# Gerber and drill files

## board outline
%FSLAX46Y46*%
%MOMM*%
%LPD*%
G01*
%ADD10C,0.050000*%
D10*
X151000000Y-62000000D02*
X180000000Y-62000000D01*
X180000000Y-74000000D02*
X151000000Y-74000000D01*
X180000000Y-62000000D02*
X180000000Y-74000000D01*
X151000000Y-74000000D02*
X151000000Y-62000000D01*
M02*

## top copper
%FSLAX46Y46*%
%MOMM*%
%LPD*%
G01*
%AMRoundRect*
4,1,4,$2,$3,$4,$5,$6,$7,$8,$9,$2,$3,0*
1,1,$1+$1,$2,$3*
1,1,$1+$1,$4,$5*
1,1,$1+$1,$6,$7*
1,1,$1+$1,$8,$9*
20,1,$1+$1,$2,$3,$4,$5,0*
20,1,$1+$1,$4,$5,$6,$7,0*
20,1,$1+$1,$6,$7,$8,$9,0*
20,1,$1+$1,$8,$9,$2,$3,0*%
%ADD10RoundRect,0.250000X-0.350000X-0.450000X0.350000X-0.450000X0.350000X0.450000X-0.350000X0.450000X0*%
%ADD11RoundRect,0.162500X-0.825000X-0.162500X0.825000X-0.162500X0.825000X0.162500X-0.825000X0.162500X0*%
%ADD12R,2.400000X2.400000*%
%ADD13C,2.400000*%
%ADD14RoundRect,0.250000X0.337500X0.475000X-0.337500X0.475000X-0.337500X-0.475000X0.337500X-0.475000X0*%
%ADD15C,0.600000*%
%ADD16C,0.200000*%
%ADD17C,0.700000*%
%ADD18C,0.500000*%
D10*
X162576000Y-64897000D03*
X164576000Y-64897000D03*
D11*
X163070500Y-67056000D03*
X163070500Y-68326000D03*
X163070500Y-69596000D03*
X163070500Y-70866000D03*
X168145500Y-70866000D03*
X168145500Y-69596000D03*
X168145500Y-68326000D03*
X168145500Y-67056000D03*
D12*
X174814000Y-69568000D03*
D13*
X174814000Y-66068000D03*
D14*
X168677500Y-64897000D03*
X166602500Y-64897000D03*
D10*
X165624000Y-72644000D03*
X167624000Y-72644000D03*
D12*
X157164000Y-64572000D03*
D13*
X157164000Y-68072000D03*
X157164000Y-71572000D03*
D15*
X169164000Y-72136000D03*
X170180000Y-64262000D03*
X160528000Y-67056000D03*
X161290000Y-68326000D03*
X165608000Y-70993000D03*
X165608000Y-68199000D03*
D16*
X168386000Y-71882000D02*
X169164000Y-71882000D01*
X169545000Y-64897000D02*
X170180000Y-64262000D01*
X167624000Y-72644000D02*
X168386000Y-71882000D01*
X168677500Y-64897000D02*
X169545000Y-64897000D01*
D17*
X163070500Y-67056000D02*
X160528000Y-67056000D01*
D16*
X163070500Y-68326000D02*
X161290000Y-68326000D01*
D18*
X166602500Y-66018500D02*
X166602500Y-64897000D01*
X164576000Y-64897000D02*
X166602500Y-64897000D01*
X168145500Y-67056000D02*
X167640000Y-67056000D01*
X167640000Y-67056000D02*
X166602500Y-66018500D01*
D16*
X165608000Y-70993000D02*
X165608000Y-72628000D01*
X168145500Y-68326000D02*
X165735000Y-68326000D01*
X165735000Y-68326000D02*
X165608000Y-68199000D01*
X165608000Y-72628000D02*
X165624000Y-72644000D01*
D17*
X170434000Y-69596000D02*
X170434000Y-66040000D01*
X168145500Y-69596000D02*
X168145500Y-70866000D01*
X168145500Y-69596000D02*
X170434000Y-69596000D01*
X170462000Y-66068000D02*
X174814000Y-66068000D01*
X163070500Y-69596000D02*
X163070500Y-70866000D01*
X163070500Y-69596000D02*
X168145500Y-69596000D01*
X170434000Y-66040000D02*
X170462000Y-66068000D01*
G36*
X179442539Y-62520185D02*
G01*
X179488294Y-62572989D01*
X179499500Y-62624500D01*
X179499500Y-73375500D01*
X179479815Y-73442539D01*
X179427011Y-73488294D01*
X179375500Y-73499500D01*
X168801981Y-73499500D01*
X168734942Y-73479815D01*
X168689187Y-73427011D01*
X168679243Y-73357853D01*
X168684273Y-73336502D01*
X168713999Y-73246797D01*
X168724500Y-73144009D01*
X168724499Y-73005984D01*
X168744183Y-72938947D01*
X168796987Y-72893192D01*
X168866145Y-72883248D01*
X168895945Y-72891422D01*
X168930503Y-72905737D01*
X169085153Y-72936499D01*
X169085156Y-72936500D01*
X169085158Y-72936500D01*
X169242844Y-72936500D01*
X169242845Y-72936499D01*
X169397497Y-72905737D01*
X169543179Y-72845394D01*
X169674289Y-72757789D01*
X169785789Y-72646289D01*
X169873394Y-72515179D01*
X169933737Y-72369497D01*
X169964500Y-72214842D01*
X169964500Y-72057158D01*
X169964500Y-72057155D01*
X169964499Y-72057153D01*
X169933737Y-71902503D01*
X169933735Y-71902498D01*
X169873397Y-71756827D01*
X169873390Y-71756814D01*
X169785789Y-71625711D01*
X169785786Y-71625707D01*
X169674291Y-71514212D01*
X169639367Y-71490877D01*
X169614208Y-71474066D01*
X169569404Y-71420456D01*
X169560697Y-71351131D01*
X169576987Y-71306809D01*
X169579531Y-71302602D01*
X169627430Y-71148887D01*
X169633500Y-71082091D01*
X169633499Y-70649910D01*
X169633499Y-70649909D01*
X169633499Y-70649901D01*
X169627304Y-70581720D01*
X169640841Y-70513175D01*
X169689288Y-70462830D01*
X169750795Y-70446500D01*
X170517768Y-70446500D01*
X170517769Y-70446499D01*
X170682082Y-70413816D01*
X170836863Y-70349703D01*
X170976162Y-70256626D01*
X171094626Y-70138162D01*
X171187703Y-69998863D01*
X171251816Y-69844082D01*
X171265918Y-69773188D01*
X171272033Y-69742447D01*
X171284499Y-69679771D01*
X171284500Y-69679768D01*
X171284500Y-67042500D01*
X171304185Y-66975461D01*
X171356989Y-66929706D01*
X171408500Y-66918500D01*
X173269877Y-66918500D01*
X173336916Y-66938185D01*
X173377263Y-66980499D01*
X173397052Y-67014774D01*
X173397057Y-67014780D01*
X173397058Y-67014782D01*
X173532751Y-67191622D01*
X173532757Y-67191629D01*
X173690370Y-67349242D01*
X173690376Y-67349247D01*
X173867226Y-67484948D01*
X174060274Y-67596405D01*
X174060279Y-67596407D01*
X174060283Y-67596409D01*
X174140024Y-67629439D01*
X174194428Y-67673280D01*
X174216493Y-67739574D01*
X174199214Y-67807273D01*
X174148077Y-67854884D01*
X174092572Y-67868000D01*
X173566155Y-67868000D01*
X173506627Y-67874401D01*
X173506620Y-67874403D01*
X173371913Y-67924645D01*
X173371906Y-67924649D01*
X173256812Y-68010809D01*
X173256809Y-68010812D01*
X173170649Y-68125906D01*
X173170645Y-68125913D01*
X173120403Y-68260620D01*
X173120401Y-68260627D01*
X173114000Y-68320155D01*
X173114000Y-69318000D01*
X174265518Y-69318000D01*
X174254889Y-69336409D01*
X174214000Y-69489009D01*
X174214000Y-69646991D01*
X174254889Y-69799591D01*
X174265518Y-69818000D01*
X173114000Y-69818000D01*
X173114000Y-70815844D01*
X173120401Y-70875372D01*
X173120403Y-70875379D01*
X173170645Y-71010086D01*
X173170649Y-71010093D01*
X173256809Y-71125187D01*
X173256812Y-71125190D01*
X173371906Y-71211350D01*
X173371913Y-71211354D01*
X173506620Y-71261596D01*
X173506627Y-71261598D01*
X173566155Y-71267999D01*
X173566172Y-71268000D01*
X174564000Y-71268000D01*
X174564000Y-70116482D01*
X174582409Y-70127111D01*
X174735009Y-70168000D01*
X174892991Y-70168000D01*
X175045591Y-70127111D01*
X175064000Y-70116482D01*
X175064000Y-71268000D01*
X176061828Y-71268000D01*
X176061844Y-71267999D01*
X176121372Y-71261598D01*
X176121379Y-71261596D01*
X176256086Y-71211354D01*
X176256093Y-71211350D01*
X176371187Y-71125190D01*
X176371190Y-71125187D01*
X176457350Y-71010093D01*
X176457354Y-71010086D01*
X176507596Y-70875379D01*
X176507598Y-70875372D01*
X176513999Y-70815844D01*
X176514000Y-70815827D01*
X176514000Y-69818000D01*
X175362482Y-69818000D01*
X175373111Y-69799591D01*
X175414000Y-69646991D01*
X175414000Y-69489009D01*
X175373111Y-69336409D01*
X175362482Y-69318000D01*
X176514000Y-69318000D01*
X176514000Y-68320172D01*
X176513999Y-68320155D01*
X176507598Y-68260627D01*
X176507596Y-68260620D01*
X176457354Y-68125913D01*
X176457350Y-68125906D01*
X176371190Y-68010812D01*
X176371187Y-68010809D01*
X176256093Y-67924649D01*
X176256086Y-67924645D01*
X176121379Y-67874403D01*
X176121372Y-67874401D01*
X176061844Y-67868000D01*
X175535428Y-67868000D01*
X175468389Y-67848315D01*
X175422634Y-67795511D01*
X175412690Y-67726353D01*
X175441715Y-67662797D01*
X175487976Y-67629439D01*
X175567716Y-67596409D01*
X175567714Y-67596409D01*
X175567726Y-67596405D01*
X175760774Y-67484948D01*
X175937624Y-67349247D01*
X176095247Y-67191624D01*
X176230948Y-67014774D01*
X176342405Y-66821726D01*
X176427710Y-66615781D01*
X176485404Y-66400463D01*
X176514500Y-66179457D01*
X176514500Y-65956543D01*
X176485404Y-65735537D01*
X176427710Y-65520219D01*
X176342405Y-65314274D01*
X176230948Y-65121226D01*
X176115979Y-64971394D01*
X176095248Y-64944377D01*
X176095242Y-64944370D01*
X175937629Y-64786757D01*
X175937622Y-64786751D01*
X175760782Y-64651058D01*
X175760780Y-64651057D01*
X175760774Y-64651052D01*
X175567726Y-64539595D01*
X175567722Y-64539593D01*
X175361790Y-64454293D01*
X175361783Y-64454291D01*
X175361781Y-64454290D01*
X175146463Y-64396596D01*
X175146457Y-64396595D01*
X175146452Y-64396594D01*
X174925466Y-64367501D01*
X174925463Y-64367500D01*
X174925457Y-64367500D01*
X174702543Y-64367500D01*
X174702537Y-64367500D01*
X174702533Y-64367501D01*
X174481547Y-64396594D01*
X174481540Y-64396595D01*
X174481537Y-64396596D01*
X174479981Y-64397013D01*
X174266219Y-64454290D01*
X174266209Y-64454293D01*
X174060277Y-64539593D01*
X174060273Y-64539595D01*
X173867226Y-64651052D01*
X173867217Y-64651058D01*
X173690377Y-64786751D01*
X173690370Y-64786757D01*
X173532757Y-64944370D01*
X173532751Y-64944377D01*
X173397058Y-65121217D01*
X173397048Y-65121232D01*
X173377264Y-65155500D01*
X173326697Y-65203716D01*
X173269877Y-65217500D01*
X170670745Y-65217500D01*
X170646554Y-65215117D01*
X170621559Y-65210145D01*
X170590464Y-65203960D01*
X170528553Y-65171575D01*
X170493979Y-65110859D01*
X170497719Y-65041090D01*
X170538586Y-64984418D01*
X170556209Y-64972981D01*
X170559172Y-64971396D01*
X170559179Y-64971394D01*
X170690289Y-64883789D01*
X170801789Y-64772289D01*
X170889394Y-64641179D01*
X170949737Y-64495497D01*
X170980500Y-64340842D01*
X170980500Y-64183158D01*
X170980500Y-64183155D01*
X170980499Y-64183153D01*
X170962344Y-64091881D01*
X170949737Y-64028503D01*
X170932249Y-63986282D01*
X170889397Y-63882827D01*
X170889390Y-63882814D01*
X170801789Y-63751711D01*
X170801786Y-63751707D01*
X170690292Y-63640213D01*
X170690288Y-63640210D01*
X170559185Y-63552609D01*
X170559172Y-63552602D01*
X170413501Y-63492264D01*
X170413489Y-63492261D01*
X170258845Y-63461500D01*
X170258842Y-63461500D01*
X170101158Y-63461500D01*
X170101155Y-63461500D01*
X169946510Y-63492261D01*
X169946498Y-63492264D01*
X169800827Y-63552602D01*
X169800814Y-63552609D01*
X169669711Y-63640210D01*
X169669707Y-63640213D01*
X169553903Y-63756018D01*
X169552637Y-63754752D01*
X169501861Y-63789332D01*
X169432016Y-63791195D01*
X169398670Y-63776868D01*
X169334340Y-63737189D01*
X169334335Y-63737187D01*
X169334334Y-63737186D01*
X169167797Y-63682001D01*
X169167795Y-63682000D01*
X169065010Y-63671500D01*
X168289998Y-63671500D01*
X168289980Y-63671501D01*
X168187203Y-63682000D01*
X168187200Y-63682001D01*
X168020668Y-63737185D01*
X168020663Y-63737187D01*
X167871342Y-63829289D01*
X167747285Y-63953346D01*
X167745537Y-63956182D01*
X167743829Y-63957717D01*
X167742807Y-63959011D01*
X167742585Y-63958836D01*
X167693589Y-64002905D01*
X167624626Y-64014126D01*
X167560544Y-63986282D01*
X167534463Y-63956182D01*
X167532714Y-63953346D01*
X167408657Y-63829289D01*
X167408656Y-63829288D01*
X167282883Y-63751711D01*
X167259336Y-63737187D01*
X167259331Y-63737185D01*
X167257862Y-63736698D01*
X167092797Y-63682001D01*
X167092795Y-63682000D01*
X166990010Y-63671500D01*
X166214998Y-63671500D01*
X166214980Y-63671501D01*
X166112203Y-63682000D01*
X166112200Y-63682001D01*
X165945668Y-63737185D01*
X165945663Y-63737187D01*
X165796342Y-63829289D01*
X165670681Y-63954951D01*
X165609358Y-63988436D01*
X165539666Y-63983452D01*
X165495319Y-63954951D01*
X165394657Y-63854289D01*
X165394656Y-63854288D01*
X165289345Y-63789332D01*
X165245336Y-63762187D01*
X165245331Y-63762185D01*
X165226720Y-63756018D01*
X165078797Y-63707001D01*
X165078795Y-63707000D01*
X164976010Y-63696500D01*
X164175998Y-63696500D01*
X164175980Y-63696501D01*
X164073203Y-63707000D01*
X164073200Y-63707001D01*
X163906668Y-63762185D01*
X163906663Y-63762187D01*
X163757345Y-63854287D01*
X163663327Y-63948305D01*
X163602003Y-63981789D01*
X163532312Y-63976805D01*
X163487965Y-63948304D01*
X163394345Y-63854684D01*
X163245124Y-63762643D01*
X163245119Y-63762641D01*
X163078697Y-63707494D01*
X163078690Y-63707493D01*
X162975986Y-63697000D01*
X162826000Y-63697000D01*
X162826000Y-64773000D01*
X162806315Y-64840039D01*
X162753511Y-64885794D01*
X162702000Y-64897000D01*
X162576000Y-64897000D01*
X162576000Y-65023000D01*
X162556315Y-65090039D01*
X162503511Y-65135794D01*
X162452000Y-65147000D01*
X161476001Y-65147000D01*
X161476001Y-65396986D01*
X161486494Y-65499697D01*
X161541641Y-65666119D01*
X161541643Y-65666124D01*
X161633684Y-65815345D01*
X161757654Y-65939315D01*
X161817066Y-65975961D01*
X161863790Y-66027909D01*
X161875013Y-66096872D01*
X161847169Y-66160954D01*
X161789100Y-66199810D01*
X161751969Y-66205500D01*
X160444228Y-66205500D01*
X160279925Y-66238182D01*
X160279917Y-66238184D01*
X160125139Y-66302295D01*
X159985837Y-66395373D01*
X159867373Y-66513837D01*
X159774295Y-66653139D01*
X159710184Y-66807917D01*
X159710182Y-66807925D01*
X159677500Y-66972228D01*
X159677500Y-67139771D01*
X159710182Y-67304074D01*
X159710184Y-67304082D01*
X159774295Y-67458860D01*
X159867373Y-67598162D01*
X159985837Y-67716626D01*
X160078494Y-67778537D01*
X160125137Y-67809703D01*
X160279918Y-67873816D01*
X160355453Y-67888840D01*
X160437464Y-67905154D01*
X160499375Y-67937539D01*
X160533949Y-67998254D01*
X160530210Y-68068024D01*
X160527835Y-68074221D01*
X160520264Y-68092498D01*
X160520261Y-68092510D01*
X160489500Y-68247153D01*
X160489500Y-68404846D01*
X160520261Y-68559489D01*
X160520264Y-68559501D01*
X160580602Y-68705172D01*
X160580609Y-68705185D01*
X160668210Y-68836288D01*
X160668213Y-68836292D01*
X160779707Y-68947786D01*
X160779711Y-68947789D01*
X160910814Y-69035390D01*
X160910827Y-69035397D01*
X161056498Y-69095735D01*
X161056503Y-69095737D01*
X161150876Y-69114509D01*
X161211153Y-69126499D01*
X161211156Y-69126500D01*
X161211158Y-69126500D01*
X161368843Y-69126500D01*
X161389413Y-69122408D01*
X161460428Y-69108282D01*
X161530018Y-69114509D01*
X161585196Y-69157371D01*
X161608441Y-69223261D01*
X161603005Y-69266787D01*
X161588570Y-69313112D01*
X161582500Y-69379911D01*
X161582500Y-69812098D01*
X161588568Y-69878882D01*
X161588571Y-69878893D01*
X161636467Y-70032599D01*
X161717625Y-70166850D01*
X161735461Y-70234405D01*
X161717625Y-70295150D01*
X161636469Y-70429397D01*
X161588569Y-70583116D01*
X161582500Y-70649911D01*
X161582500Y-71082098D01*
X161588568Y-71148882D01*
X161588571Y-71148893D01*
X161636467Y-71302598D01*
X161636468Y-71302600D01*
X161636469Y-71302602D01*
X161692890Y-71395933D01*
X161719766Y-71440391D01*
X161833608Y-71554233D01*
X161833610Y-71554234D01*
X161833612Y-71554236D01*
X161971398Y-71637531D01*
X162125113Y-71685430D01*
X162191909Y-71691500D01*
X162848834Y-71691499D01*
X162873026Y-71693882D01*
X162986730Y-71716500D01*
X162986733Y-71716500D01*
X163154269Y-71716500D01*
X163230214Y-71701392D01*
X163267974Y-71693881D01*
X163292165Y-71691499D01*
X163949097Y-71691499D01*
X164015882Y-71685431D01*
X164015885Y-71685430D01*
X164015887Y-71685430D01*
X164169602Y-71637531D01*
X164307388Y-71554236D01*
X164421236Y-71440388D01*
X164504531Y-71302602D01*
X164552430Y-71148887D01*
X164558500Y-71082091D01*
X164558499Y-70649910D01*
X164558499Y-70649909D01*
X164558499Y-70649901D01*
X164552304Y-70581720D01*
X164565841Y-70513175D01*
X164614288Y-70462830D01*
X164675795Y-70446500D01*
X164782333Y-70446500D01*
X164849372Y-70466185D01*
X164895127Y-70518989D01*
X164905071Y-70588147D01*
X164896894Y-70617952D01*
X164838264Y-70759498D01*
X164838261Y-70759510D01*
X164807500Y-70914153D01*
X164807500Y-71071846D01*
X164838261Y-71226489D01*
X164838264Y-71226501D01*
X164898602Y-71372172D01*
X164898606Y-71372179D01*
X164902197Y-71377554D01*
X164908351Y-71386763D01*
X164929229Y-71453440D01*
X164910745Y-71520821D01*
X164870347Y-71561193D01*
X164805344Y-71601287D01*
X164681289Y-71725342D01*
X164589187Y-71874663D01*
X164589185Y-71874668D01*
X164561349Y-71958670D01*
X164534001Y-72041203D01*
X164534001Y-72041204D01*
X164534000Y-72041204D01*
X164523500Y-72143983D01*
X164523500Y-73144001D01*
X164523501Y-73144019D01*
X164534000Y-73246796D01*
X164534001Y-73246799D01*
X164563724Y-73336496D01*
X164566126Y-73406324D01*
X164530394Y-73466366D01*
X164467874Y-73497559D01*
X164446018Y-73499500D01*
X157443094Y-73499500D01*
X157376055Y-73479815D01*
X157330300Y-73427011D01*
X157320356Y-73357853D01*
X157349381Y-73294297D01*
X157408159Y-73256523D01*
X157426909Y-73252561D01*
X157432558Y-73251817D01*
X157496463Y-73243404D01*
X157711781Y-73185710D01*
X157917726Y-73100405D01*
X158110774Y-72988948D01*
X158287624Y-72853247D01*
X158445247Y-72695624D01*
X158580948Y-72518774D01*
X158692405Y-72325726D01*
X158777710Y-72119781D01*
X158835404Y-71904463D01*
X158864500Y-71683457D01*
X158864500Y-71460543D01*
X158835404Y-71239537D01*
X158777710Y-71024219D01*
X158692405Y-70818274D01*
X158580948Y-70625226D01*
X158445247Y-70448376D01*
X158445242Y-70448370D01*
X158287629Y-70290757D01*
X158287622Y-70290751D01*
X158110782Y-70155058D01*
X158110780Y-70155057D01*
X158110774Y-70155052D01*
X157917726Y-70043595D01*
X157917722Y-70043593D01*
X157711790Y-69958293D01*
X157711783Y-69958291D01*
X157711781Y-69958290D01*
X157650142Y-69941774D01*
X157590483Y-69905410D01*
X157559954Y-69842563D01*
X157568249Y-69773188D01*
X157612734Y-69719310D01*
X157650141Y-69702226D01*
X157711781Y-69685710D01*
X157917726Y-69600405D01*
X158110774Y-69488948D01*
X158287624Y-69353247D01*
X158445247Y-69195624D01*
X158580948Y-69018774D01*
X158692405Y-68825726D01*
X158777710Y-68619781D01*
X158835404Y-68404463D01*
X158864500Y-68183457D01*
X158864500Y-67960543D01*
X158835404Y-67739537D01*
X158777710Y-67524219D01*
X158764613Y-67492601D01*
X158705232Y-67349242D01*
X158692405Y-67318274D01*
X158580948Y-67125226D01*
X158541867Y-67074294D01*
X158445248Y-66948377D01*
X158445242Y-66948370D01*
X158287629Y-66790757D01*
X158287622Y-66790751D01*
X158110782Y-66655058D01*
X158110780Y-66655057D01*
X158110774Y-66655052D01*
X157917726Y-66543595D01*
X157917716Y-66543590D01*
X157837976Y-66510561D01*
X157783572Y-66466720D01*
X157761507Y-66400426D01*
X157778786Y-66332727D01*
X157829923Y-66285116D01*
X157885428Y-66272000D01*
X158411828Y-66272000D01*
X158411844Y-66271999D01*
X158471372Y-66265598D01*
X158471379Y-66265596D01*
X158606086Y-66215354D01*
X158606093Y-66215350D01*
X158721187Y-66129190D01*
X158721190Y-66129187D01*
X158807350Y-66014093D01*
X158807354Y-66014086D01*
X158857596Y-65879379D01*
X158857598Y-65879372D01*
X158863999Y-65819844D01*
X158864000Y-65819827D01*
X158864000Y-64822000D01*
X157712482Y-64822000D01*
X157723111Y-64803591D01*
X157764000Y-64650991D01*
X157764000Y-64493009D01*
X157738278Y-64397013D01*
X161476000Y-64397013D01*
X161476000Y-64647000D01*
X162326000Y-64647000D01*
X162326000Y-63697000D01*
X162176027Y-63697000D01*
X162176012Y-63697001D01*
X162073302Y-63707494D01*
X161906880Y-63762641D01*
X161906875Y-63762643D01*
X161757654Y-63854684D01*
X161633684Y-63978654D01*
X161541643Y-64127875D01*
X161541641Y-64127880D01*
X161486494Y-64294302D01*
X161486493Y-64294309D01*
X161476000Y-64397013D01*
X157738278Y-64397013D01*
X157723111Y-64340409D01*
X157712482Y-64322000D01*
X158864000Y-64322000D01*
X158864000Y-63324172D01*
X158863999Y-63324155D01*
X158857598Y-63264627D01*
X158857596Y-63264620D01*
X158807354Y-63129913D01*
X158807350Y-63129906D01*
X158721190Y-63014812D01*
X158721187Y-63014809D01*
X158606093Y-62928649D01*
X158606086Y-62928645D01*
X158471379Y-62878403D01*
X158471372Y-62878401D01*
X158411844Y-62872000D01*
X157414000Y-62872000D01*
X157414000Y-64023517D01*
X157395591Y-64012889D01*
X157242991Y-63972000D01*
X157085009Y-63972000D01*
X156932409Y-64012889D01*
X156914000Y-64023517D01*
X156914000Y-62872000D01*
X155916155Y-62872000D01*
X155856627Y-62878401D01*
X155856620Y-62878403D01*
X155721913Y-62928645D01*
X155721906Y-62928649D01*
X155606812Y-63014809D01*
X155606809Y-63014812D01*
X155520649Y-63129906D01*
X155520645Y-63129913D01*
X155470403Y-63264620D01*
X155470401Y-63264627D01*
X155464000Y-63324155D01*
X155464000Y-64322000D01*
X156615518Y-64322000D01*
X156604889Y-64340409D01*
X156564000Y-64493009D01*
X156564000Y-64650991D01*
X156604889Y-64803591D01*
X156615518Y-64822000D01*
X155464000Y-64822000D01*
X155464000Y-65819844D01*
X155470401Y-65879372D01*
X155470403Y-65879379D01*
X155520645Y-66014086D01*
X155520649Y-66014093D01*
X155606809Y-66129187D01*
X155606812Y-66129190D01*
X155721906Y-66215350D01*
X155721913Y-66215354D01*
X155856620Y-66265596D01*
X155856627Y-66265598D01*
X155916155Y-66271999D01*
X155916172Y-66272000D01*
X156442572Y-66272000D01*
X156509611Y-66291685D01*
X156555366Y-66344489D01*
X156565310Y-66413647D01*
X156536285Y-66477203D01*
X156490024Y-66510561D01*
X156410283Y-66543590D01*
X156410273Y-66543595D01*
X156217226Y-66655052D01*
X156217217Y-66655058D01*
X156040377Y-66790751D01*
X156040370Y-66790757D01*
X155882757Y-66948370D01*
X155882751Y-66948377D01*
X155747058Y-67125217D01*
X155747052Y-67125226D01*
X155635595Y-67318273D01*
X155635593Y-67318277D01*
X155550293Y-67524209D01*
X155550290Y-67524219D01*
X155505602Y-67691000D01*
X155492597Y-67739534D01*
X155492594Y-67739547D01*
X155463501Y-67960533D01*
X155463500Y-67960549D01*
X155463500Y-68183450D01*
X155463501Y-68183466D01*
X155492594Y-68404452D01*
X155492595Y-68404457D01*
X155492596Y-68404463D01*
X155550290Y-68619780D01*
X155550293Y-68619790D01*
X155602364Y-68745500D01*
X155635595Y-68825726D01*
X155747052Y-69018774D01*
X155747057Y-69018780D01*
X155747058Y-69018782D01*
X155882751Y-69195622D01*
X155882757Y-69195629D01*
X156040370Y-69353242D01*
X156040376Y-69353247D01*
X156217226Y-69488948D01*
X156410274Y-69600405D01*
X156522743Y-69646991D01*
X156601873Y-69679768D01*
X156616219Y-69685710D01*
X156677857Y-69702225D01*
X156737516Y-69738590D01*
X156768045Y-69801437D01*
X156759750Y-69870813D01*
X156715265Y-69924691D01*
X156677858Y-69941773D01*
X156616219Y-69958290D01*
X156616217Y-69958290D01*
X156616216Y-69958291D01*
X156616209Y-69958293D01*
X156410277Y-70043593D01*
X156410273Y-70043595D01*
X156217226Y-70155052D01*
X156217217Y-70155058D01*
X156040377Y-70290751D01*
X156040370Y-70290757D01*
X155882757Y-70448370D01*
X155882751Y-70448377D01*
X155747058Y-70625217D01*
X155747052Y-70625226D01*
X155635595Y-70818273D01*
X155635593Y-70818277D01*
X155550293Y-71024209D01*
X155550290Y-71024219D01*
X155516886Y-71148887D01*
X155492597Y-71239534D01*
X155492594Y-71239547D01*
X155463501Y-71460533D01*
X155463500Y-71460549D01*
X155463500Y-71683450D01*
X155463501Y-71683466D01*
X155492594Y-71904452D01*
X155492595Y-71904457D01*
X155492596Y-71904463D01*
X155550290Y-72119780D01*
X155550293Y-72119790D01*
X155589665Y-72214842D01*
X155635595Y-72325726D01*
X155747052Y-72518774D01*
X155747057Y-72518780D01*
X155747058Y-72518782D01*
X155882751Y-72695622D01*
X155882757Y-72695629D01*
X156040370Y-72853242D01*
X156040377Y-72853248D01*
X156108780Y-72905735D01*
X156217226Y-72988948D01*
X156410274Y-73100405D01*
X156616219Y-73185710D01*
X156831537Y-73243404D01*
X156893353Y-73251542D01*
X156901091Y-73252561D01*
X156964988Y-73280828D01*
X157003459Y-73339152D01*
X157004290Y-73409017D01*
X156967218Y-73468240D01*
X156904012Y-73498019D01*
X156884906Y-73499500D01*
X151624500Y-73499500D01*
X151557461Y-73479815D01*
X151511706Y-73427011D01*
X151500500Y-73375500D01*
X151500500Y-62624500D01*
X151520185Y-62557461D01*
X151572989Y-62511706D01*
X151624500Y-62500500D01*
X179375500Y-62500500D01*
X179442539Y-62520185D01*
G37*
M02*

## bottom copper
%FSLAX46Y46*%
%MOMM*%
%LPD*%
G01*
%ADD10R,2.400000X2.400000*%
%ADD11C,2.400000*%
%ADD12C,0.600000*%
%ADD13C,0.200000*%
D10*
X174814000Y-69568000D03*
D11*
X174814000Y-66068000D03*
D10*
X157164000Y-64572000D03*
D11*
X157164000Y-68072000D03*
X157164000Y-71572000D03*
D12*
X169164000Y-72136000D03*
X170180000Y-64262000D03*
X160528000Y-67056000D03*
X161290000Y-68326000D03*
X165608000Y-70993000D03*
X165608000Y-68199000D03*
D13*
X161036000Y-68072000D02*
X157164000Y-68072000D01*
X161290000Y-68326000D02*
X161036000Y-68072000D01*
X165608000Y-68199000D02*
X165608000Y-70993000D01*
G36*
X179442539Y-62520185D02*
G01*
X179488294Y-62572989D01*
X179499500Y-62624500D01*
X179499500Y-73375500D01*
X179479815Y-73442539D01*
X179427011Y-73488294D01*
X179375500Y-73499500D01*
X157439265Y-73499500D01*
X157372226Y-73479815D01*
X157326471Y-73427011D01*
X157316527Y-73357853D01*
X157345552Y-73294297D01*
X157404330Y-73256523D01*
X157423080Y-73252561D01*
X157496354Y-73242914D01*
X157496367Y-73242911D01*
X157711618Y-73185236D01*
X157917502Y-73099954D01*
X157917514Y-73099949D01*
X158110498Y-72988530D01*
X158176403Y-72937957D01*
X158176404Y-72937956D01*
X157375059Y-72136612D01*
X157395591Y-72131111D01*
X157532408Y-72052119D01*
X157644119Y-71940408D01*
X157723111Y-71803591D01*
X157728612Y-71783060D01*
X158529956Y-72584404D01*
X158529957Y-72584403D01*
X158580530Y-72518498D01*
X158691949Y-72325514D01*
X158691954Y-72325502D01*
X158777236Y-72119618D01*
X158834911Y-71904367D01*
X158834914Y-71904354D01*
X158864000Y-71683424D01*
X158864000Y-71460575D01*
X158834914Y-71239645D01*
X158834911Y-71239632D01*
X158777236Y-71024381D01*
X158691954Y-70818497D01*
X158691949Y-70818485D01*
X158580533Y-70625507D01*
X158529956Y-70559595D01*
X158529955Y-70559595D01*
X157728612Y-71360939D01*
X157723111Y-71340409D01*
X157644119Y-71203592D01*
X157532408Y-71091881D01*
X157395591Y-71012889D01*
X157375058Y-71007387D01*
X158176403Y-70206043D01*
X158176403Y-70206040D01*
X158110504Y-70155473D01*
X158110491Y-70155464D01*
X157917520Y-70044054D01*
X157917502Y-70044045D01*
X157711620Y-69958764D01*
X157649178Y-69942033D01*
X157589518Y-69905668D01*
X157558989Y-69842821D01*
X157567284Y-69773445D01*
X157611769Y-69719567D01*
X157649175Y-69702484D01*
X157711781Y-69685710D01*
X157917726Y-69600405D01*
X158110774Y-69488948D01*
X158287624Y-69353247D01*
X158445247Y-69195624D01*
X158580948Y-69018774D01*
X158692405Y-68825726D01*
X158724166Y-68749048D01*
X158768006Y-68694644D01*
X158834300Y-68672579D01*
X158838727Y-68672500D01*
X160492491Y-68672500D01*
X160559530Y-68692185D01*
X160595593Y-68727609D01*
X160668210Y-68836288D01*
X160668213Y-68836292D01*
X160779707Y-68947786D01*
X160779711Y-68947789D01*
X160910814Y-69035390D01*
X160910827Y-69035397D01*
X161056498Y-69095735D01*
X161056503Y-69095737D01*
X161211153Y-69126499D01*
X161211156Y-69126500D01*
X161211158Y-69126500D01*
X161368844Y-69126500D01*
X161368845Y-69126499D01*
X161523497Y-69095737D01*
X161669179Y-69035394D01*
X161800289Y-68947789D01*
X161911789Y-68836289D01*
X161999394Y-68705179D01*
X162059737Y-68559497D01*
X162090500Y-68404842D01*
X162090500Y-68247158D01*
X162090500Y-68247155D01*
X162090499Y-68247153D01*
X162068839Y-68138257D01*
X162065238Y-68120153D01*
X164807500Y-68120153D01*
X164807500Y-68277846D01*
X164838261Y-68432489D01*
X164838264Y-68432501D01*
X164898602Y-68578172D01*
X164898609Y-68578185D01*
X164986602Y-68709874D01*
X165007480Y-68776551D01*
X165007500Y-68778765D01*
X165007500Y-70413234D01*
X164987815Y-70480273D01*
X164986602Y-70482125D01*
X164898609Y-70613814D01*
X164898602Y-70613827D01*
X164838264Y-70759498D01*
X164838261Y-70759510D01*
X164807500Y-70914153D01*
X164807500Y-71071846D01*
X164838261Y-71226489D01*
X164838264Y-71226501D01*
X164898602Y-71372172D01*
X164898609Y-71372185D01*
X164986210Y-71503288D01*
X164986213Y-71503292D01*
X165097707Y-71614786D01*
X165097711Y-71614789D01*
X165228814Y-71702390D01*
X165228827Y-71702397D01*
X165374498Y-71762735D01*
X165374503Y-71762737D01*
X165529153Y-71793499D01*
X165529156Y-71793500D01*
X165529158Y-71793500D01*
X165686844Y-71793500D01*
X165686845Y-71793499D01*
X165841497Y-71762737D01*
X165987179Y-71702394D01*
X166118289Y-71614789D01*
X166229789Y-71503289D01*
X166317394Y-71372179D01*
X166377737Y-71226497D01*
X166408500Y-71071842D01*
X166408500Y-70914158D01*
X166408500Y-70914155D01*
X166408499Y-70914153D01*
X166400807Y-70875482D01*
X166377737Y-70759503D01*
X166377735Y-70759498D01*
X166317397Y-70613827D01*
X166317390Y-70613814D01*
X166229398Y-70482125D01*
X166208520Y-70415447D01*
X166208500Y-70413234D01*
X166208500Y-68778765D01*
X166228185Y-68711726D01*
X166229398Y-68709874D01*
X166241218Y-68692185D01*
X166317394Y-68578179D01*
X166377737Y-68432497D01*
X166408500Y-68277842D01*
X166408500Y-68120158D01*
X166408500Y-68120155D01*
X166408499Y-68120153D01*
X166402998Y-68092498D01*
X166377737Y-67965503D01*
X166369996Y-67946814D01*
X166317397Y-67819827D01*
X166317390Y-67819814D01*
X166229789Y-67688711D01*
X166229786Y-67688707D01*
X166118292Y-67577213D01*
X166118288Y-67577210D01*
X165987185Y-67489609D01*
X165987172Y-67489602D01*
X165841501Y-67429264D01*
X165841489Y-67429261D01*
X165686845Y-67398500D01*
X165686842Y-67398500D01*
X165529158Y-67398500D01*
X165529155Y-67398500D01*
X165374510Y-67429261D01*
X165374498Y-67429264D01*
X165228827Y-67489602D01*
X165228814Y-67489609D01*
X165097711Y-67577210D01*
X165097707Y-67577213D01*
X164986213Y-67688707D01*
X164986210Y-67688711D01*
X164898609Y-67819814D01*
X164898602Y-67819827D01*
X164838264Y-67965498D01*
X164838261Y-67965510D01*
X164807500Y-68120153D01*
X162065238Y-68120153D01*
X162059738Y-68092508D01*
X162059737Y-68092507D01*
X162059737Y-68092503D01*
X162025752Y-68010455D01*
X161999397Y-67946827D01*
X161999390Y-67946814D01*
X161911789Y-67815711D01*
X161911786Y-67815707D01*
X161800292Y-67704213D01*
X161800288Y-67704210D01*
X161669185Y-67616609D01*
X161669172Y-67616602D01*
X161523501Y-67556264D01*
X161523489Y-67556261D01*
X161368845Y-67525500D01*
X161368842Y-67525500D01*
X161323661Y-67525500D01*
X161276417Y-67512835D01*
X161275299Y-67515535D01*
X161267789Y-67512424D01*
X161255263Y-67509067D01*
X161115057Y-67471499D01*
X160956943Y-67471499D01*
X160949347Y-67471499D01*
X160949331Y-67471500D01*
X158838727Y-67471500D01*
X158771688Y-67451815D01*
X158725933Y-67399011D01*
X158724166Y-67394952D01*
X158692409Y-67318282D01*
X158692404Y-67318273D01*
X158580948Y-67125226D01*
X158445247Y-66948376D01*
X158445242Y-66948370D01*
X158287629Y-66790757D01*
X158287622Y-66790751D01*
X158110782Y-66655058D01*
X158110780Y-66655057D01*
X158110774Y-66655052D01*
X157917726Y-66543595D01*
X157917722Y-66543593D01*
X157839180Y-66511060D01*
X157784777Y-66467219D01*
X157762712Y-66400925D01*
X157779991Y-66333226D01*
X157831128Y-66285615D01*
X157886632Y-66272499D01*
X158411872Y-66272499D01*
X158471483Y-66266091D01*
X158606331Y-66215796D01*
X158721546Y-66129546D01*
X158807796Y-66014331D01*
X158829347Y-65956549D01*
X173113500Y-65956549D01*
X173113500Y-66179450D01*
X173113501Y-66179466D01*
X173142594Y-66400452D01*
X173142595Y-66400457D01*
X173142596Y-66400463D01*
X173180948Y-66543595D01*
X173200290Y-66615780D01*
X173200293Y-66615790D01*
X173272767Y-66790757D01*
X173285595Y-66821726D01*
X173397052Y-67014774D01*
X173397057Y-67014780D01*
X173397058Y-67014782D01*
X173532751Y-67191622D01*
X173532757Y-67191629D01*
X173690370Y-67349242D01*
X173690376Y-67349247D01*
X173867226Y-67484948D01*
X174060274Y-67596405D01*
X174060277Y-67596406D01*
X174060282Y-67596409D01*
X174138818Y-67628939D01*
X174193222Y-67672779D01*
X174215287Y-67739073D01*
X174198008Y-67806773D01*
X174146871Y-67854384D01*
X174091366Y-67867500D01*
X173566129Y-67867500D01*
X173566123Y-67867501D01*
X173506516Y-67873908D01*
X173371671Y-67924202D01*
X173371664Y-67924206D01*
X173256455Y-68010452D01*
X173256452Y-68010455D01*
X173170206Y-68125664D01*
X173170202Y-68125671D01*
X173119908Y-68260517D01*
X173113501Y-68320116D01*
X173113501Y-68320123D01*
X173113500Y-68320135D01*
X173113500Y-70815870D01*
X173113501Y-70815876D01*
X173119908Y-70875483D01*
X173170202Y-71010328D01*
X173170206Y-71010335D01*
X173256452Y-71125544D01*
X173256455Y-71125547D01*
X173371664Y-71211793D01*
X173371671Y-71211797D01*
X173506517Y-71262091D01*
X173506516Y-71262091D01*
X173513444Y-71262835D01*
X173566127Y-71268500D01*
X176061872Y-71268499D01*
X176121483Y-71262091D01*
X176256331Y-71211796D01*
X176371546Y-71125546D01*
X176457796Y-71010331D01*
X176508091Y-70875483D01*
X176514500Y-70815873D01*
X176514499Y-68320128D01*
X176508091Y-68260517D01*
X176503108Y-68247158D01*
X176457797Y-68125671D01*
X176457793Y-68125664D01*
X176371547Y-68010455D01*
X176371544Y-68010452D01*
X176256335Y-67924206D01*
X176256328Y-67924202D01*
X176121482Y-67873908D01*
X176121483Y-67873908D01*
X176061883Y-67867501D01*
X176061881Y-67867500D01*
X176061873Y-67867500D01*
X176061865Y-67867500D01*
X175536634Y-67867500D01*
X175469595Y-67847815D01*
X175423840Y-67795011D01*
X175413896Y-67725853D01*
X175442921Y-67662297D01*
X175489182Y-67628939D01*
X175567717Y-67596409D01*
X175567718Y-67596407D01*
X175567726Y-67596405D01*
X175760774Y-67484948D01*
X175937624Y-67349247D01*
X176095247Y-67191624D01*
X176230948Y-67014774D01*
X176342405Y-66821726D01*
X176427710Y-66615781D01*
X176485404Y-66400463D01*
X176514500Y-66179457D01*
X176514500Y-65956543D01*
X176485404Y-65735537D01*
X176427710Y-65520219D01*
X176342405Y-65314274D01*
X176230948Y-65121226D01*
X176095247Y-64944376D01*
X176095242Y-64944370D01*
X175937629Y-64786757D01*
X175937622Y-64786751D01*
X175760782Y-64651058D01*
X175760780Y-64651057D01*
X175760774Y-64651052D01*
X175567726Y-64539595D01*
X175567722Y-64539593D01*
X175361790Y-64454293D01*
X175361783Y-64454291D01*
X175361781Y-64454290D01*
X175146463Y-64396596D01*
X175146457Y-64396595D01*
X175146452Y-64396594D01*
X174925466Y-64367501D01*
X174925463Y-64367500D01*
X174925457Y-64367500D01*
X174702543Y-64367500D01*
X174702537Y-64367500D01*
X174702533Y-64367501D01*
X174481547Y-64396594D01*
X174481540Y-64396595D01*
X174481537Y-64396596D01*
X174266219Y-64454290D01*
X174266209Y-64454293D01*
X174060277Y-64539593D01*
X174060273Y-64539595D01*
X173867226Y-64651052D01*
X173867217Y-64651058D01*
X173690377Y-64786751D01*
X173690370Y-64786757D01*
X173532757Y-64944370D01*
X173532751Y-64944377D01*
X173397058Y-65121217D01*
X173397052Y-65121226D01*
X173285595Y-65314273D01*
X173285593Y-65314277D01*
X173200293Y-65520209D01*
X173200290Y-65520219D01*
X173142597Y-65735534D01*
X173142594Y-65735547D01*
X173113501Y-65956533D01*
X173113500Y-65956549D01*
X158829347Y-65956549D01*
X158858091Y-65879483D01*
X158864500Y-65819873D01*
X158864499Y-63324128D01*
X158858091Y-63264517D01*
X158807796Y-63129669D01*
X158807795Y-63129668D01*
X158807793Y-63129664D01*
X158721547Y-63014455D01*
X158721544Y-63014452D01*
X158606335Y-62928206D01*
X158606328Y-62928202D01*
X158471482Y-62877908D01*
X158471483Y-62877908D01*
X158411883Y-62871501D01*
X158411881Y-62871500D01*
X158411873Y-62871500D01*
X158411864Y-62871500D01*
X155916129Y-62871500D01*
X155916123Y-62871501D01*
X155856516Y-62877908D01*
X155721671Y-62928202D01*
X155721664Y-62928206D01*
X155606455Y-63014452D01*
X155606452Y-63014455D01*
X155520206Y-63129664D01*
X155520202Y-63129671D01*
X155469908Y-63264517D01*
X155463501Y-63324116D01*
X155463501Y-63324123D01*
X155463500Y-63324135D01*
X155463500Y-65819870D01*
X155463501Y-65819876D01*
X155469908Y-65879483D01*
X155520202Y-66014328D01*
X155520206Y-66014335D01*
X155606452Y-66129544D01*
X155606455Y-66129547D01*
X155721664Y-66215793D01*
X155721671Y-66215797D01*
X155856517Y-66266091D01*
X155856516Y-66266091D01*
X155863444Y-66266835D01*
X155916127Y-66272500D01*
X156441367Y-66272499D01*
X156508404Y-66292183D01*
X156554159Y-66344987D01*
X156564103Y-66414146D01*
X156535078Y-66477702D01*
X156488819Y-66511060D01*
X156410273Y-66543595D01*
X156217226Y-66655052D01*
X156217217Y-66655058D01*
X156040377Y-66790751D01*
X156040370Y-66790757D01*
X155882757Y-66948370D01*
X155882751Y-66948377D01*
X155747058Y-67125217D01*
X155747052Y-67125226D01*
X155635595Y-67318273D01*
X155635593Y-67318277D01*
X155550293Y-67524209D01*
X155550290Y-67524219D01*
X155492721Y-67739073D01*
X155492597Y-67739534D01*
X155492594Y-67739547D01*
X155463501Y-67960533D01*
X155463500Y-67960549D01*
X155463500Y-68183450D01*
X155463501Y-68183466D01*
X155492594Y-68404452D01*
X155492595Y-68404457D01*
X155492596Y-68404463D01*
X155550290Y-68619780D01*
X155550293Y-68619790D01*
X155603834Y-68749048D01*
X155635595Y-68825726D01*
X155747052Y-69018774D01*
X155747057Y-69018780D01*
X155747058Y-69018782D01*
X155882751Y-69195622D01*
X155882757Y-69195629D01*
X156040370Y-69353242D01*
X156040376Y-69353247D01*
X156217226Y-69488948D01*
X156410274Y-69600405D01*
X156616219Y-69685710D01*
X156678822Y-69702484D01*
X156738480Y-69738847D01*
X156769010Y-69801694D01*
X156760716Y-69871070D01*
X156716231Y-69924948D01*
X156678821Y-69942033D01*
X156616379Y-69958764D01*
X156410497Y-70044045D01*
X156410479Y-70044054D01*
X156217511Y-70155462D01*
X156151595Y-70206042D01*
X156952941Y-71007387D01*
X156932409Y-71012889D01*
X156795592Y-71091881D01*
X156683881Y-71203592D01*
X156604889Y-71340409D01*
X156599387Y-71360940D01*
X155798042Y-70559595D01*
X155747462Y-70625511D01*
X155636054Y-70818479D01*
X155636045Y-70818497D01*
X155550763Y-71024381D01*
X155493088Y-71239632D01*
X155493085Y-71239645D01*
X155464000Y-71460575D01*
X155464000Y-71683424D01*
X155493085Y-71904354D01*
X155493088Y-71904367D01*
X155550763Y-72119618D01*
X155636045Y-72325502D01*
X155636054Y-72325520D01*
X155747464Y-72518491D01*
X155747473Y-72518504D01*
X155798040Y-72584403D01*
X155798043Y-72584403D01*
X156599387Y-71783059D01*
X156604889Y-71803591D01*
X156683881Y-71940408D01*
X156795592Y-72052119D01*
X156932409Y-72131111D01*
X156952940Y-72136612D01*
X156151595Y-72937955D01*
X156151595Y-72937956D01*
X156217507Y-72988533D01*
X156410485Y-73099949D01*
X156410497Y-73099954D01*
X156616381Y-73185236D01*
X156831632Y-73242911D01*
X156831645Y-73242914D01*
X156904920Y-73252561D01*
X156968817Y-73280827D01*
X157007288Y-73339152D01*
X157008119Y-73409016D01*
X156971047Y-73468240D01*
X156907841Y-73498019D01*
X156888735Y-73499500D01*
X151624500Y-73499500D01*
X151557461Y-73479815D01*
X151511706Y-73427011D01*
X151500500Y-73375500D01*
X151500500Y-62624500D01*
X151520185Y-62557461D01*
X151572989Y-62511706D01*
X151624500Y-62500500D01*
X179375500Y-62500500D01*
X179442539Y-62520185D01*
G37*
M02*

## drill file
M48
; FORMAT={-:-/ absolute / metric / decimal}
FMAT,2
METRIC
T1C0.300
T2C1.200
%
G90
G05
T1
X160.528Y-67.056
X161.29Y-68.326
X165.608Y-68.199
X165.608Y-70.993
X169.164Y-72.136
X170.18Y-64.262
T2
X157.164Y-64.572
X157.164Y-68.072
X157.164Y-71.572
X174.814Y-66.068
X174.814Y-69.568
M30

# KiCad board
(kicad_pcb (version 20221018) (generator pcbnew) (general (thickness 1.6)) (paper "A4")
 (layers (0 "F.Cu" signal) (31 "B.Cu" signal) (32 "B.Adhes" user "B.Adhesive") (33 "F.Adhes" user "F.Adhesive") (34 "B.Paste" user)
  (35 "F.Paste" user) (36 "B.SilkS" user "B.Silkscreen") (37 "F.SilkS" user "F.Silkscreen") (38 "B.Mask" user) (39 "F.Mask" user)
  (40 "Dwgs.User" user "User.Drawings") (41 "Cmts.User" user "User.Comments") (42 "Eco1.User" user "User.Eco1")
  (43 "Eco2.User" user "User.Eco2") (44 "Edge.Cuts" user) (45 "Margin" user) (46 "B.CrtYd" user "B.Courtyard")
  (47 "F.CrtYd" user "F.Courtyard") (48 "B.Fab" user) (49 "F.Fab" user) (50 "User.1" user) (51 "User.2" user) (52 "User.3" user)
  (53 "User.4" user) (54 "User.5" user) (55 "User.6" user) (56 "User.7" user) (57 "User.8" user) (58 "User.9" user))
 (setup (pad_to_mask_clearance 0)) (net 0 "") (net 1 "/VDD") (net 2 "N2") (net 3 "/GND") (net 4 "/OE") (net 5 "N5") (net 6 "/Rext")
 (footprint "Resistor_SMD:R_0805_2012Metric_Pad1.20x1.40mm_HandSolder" (layer "F.Cu") (at 163.576 64.897)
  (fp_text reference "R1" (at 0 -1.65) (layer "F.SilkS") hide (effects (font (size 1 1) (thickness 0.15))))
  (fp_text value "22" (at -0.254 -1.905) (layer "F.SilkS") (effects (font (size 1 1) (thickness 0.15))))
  (pad "1" smd roundrect (at -1 0) (size 1.2 1.4) (layers "F.Cu" "F.Paste" "F.Mask") (roundrect_rratio 0.2083333333) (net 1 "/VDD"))
  (pad "2" smd roundrect (at 1 0) (size 1.2 1.4) (layers "F.Cu" "F.Paste" "F.Mask") (roundrect_rratio 0.2083333333) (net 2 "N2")))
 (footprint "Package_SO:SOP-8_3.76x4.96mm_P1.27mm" (layer "F.Cu") (at 165.608 68.961)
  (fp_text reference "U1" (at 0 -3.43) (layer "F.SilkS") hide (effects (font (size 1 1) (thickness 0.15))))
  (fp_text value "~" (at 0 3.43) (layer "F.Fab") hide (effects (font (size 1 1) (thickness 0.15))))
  (pad "1" smd roundrect (at -2.5375 -1.905) (size 1.975 0.65) (layers "F.Cu" "F.Paste" "F.Mask") (roundrect_rratio 0.25) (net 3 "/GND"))
  (pad "2" smd roundrect (at -2.5375 -0.635) (size 1.975 0.65) (layers "F.Cu" "F.Paste" "F.Mask") (roundrect_rratio 0.25) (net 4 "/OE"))
  (pad "3" smd roundrect (at -2.5375 0.635) (size 1.975 0.65) (layers "F.Cu" "F.Paste" "F.Mask") (roundrect_rratio 0.25) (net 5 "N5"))
  (pad "4" smd roundrect (at -2.5375 1.905) (size 1.975 0.65) (layers "F.Cu" "F.Paste" "F.Mask") (roundrect_rratio 0.25) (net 5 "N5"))
  (pad "5" smd roundrect (at 2.5375 1.905) (size 1.975 0.65) (layers "F.Cu" "F.Paste" "F.Mask") (roundrect_rratio 0.25) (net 5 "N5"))
  (pad "6" smd roundrect (at 2.5375 0.635) (size 1.975 0.65) (layers "F.Cu" "F.Paste" "F.Mask") (roundrect_rratio 0.25) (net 5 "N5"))
  (pad "7" smd roundrect (at 2.5375 -0.635) (size 1.975 0.65) (layers "F.Cu" "F.Paste" "F.Mask") (roundrect_rratio 0.25) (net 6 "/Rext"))
  (pad "8" smd roundrect (at 2.5375 -1.905) (size 1.975 0.65) (layers "F.Cu" "F.Paste" "F.Mask") (roundrect_rratio 0.25) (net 2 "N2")))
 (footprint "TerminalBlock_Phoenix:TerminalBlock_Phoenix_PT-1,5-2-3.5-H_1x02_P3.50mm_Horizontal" (layer "F.Cu") (at 174.814 69.568 90)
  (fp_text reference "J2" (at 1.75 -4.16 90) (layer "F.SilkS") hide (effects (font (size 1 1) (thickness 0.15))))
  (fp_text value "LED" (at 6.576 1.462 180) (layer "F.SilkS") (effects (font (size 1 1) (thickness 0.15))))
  (pad "1" thru_hole rect (at 0 0 90) (size 2.4 2.4) (drill 1.2) (layers "*.Cu" "*.Mask") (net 1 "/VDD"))
  (pad "2" thru_hole circle (at 3.5 0 90) (size 2.4 2.4) (drill 1.2) (layers "*.Cu" "*.Mask") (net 5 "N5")))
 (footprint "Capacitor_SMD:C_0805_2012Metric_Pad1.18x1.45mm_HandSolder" (layer "F.Cu") (at 167.64 64.897 180)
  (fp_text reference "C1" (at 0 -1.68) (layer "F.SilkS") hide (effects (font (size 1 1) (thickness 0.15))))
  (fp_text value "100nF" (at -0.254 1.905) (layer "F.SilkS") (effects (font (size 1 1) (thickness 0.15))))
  (pad "1" smd roundrect (at -1.0375 0 180) (size 1.175 1.45) (layers "F.Cu" "F.Paste" "F.Mask") (roundrect_rratio 0.2127659574)
   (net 3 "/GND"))
  (pad "2" smd roundrect (at 1.0375 0 180) (size 1.175 1.45) (layers "F.Cu" "F.Paste" "F.Mask") (roundrect_rratio 0.2127659574) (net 2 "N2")))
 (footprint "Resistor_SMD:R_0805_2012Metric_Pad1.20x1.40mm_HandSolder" (layer "F.Cu") (at 166.624 72.644)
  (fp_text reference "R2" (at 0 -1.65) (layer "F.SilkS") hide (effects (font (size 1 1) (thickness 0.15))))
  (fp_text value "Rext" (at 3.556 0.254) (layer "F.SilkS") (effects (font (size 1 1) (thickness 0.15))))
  (pad "1" smd roundrect (at -1 0) (size 1.2 1.4) (layers "F.Cu" "F.Paste" "F.Mask") (roundrect_rratio 0.2083333333) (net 6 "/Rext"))
  (pad "2" smd roundrect (at 1 0) (size 1.2 1.4) (layers "F.Cu" "F.Paste" "F.Mask") (roundrect_rratio 0.2083333333) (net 3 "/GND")))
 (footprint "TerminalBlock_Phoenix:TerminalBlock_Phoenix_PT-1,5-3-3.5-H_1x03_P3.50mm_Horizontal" (layer "F.Cu") (at 157.164 64.572 -90)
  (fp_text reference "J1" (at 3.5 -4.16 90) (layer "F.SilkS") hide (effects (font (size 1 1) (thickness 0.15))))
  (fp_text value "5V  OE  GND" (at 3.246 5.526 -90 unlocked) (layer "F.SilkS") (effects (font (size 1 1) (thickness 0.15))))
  (pad "1" thru_hole rect (at 0 0 270) (size 2.4 2.4) (drill 1.2) (layers "*.Cu" "*.Mask") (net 1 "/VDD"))
  (pad "2" thru_hole circle (at 3.5 0 270) (size 2.4 2.4) (drill 1.2) (layers "*.Cu" "*.Mask") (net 4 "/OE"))
  (pad "3" thru_hole circle (at 7 0 270) (size 2.4 2.4) (drill 1.2) (layers "*.Cu" "*.Mask") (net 3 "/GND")))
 (gr_line (start 151 62) (end 180 62) (stroke (width 0.05) (type default)) (layer "Edge.Cuts"))
 (gr_line (start 180 74) (end 151 74) (stroke (width 0.05) (type default)) (layer "Edge.Cuts"))
 (gr_line (start 180 62) (end 180 74) (stroke (width 0.05) (type default)) (layer "Edge.Cuts"))
 (gr_line (start 151 74) (end 151 62) (stroke (width 0.05) (type default)) (layer "Edge.Cuts"))
 (segment (start 168.386 71.882) (end 169.164 71.882) (width 0.2) (layer "F.Cu") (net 3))
 (segment (start 169.545 64.897) (end 170.18 64.262) (width 0.2) (layer "F.Cu") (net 3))
 (segment (start 167.624 72.644) (end 168.386 71.882) (width 0.2) (layer "F.Cu") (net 3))
 (segment (start 168.6775 64.897) (end 169.545 64.897) (width 0.2) (layer "F.Cu") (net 3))
 (segment (start 163.0705 67.056) (end 160.528 67.056) (width 0.7) (layer "F.Cu") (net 3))
 (via (at 169.164 72.136) (size 0.6) (drill 0.3) (layers "F.Cu" "B.Cu") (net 3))
 (via (at 170.18 64.262) (size 0.6) (drill 0.3) (layers "F.Cu" "B.Cu") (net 3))
 (via (at 160.528 67.056) (size 0.6) (drill 0.3) (layers "F.Cu" "B.Cu") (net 3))
 (segment (start 163.0705 68.326) (end 161.29 68.326) (width 0.2) (layer "F.Cu") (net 4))
 (via (at 161.29 68.326) (size 0.6) (drill 0.3) (layers "F.Cu" "B.Cu") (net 4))
 (segment (start 161.036 68.072) (end 157.164 68.072) (width 0.2) (layer "B.Cu") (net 4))
 (segment (start 161.29 68.326) (end 161.036 68.072) (width 0.2) (layer "B.Cu") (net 4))
 (segment (start 166.6025 66.0185) (end 166.6025 64.897) (width 0.5) (layer "F.Cu") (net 2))
 (segment (start 164.576 64.897) (end 166.6025 64.897) (width 0.5) (layer "F.Cu") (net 2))
 (segment (start 168.1455 67.056) (end 167.64 67.056) (width 0.5) (layer "F.Cu") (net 2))
 (segment (start 167.64 67.056) (end 166.6025 66.0185) (width 0.5) (layer "F.Cu") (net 2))
 (segment (start 165.608 70.993) (end 165.608 72.628) (width 0.2) (layer "F.Cu") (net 6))
 (segment (start 168.1455 68.326) (end 165.735 68.326) (width 0.2) (layer "F.Cu") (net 6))
 (segment (start 165.735 68.326) (end 165.608 68.199) (width 0.2) (layer "F.Cu") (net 6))
 (segment (start 165.608 72.628) (end 165.624 72.644) (width 0.2) (layer "F.Cu") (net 6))
 (via (at 165.608 70.993) (size 0.6) (drill 0.3) (layers "F.Cu" "B.Cu") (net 6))
 (via (at 165.608 68.199) (size 0.6) (drill 0.3) (layers "F.Cu" "B.Cu") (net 6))
 (segment (start 165.608 68.199) (end 165.608 70.993) (width 0.2) (layer "B.Cu") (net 6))
 (segment (start 170.434 69.596) (end 170.434 66.04) (width 0.7) (layer "F.Cu") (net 5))
 (segment (start 168.1455 69.596) (end 168.1455 70.866) (width 0.7) (layer "F.Cu") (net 5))
 (segment (start 168.1455 69.596) (end 170.434 69.596) (width 0.7) (layer "F.Cu") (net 5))
 (segment (start 170.462 66.068) (end 174.814 66.068) (width 0.7) (layer "F.Cu") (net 5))
 (segment (start 163.0705 69.596) (end 163.0705 70.866) (width 0.7) (layer "F.Cu") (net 5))
 (segment (start 163.0705 69.596) (end 168.1455 69.596) (width 0.7) (layer "F.Cu") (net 5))
 (segment (start 170.434 66.04) (end 170.462 66.068) (width 0.7) (layer "F.Cu") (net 5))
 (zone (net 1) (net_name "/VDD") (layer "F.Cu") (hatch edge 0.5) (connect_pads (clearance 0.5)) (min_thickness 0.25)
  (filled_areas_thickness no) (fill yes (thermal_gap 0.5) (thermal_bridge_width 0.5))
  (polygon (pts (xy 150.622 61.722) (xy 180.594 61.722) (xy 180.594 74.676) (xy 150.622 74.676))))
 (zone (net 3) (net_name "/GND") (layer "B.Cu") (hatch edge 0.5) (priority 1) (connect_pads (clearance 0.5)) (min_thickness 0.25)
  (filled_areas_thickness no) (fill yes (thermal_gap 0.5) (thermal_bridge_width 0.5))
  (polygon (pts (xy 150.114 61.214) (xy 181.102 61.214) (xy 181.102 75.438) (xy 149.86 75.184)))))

